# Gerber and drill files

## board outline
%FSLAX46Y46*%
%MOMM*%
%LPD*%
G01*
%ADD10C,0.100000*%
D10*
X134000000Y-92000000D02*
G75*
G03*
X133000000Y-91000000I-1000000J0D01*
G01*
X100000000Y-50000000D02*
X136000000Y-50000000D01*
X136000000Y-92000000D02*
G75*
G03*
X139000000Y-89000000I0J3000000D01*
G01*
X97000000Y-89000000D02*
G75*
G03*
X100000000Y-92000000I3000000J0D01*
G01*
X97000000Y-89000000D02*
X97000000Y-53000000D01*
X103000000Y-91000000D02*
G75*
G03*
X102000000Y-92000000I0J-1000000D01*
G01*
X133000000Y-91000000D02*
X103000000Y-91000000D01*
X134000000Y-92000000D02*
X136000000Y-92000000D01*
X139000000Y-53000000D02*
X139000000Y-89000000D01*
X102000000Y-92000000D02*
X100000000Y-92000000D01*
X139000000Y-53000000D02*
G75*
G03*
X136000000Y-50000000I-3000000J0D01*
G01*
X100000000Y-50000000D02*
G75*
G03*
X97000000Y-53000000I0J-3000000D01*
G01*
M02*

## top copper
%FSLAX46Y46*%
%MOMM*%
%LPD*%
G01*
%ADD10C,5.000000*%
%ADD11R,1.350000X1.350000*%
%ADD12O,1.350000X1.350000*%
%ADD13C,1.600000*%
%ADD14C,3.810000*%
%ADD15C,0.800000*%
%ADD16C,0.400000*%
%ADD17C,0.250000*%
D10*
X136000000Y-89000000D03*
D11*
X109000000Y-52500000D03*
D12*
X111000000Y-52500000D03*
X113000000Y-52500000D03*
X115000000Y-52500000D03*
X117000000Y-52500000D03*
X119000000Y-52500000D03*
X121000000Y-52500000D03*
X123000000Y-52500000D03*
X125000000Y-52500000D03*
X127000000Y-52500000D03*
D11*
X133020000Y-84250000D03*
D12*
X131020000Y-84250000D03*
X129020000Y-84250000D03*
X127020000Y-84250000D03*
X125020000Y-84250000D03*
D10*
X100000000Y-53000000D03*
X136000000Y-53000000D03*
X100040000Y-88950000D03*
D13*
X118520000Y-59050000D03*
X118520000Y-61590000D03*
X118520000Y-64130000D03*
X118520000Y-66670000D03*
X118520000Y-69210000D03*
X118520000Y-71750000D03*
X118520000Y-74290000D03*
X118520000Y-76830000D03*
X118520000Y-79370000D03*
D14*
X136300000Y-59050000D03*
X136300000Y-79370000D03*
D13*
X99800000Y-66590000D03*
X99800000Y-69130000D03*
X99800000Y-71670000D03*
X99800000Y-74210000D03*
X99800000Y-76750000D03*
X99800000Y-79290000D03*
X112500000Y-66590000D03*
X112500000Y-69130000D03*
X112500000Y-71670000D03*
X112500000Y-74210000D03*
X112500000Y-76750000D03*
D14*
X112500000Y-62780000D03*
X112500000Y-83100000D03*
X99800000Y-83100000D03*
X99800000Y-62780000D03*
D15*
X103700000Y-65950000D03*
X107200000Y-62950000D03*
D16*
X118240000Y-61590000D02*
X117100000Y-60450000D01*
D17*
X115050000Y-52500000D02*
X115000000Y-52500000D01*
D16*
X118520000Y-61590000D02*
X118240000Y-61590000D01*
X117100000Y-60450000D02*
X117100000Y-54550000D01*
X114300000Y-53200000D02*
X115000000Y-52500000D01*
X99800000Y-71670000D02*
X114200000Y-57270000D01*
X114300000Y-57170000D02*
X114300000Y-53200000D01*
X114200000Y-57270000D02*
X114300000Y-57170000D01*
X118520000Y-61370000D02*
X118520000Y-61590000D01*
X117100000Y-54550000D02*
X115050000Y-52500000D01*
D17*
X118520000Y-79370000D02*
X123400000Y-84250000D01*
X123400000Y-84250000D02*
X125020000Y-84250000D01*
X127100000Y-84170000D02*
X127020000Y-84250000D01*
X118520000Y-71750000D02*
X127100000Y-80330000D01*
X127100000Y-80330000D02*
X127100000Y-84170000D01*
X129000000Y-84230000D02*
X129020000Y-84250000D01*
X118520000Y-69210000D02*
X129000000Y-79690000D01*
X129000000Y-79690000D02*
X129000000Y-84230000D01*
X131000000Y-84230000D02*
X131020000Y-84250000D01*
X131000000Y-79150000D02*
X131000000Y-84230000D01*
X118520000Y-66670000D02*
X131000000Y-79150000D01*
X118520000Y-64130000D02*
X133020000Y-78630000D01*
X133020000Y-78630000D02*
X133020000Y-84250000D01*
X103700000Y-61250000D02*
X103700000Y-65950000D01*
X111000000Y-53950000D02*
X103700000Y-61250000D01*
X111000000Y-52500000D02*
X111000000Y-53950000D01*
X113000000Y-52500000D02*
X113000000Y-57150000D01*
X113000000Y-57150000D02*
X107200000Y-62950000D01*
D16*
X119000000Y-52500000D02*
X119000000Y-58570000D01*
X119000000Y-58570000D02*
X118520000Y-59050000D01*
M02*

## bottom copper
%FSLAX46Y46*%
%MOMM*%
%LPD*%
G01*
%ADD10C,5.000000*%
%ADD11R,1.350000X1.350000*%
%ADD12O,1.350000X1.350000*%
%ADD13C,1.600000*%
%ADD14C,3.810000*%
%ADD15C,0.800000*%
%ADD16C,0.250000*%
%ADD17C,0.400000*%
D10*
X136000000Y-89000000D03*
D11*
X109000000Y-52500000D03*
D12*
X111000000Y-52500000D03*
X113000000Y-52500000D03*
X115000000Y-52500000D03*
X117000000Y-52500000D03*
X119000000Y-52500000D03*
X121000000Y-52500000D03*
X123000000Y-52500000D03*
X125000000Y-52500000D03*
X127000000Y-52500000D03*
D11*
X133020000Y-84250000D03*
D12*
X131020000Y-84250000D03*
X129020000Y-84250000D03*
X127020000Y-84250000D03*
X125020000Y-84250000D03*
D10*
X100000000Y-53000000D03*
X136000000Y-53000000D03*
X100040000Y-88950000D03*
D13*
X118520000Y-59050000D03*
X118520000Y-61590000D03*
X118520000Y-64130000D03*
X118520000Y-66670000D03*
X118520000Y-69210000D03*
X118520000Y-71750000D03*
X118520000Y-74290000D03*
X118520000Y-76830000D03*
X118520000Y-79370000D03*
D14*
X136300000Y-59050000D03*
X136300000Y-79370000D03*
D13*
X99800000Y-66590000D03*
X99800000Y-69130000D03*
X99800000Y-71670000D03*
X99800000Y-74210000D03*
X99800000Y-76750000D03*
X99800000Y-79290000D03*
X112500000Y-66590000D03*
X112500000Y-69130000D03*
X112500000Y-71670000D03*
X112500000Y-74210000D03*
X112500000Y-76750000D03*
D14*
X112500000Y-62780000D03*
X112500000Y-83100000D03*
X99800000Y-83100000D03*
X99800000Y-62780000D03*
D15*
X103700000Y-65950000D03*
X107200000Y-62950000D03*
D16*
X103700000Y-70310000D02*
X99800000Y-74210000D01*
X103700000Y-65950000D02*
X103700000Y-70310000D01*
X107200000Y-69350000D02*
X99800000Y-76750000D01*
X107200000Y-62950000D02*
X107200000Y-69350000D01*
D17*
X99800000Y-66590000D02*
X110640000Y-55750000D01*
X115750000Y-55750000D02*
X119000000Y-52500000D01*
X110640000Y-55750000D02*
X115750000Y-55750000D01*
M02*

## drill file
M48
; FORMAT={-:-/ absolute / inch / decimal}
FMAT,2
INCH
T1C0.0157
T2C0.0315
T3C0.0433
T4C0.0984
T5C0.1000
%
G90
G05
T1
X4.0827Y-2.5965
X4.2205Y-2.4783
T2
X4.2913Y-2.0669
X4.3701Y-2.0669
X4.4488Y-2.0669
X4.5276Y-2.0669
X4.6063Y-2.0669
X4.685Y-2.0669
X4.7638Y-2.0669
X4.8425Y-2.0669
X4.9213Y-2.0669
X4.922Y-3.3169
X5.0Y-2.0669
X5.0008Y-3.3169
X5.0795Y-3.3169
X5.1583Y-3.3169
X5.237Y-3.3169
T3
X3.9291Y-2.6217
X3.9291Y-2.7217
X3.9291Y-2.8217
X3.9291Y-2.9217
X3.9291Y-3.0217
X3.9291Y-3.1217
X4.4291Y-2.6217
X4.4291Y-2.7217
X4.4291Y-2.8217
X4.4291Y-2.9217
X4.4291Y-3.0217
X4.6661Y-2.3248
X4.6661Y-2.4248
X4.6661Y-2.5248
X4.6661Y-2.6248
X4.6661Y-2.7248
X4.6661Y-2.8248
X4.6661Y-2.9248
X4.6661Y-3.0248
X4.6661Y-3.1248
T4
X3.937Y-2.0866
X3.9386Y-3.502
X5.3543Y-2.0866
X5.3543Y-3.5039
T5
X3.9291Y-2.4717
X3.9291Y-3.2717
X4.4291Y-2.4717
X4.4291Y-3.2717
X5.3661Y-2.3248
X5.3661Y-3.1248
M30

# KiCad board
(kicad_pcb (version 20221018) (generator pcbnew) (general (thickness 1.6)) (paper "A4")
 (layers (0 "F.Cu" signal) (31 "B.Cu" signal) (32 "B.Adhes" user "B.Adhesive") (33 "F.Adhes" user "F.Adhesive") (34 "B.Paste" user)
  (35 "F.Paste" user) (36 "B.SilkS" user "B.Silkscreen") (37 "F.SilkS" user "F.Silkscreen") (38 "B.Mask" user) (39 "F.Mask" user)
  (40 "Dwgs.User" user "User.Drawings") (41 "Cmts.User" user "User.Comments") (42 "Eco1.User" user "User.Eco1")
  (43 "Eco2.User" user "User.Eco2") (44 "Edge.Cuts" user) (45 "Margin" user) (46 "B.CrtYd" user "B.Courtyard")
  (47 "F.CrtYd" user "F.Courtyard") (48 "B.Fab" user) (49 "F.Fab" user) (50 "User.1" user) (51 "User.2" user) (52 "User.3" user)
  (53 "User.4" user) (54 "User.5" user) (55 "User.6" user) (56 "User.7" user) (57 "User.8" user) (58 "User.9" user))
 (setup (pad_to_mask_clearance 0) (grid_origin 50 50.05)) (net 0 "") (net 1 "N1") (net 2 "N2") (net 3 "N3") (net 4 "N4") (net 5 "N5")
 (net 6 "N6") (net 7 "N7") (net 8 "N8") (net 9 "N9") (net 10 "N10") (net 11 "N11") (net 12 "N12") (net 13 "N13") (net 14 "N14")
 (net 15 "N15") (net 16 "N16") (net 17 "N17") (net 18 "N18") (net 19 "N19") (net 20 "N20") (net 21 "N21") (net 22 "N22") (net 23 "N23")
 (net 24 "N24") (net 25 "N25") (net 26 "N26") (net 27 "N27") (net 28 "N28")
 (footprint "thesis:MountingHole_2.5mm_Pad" (layer "F.Cu") (at 136.06 89)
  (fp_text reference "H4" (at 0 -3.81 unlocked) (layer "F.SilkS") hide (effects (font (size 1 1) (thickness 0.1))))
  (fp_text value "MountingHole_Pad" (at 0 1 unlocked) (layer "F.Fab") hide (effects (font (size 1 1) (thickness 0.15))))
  (pad "1" thru_hole circle (at -0.06 0) (size 5 5) (drill 2.5) (layers "*.Cu" "*.Mask") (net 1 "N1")))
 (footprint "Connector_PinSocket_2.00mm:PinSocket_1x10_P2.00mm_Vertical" (layer "F.Cu") (at 109 52.5 90)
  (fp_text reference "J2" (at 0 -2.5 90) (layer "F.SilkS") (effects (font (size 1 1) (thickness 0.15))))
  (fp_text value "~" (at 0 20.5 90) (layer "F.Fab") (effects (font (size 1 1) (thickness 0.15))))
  (pad "1" thru_hole rect (at 0 0 90) (size 1.35 1.35) (drill 0.8) (layers "*.Cu" "*.Mask") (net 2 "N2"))
  (pad "2" thru_hole oval (at 0 2 90) (size 1.35 1.35) (drill 0.8) (layers "*.Cu" "*.Mask") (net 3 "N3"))
  (pad "3" thru_hole oval (at 0 4 90) (size 1.35 1.35) (drill 0.8) (layers "*.Cu" "*.Mask") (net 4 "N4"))
  (pad "4" thru_hole oval (at 0 6 90) (size 1.35 1.35) (drill 0.8) (layers "*.Cu" "*.Mask") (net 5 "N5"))
  (pad "5" thru_hole oval (at 0 8 90) (size 1.35 1.35) (drill 0.8) (layers "*.Cu" "*.Mask") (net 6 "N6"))
  (pad "6" thru_hole oval (at 0 10 90) (size 1.35 1.35) (drill 0.8) (layers "*.Cu" "*.Mask") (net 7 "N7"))
  (pad "7" thru_hole oval (at 0 12 90) (size 1.35 1.35) (drill 0.8) (layers "*.Cu" "*.Mask") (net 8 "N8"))
  (pad "8" thru_hole oval (at 0 14 90) (size 1.35 1.35) (drill 0.8) (layers "*.Cu" "*.Mask") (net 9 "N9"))
  (pad "9" thru_hole oval (at 0 16 90) (size 1.35 1.35) (drill 0.8) (layers "*.Cu" "*.Mask") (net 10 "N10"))
  (pad "10" thru_hole oval (at 0 18 90) (size 1.35 1.35) (drill 0.8) (layers "*.Cu" "*.Mask") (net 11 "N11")))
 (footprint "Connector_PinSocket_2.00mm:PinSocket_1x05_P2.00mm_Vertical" (layer "F.Cu") (at 133.02 84.25 -90)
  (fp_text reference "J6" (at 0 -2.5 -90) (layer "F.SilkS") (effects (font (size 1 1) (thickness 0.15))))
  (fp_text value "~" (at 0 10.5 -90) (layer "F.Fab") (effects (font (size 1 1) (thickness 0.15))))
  (pad "1" thru_hole rect (at 0 0 270) (size 1.35 1.35) (drill 0.8) (layers "*.Cu" "*.Mask") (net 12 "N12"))
  (pad "2" thru_hole oval (at 0 2 270) (size 1.35 1.35) (drill 0.8) (layers "*.Cu" "*.Mask") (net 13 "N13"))
  (pad "3" thru_hole oval (at 0 4 270) (size 1.35 1.35) (drill 0.8) (layers "*.Cu" "*.Mask") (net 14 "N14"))
  (pad "4" thru_hole oval (at 0 6 270) (size 1.35 1.35) (drill 0.8) (layers "*.Cu" "*.Mask") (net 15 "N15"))
  (pad "5" thru_hole oval (at 0 8 270) (size 1.35 1.35) (drill 0.8) (layers "*.Cu" "*.Mask") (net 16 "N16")))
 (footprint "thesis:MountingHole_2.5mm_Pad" (layer "F.Cu") (at 100.06 53)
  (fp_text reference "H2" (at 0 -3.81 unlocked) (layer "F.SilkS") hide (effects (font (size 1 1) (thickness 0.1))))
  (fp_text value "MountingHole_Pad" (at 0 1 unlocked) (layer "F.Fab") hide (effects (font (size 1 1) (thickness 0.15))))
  (pad "1" thru_hole circle (at -0.06 0) (size 5 5) (drill 2.5) (layers "*.Cu" "*.Mask") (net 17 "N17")))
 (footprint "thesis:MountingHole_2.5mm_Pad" (layer "F.Cu") (at 136.06 53)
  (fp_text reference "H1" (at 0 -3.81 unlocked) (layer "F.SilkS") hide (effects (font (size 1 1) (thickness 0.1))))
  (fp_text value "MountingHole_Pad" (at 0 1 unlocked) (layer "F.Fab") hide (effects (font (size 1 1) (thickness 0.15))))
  (pad "1" thru_hole circle (at -0.06 0) (size 5 5) (drill 2.5) (layers "*.Cu" "*.Mask") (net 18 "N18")))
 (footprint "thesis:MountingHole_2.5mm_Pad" (layer "F.Cu") (at 100.1 88.95)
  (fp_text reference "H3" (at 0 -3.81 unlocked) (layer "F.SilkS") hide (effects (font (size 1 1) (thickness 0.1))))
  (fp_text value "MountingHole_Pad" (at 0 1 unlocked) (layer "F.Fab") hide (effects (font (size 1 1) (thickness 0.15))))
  (pad "1" thru_hole circle (at -0.06 0) (size 5 5) (drill 2.5) (layers "*.Cu" "*.Mask") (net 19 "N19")))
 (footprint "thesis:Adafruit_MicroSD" (layer "F.Cu") (at 138.84 56.51 -90)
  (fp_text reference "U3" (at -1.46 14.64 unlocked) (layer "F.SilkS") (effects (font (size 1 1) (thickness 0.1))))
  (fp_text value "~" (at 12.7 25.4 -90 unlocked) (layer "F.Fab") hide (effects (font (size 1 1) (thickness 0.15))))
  (pad "1" thru_hole circle (at 2.54 20.32 270) (size 1.6 1.6) (drill 1.1) (layers "*.Cu" "*.Mask") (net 7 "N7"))
  (pad "2" thru_hole circle (at 5.08 20.32 270) (size 1.6 1.6) (drill 1.1) (layers "*.Cu" "*.Mask") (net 5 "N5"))
  (pad "3" thru_hole circle (at 7.62 20.32 270) (size 1.6 1.6) (drill 1.1) (layers "*.Cu" "*.Mask") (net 12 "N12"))
  (pad "4" thru_hole circle (at 10.16 20.32 270) (size 1.6 1.6) (drill 1.1) (layers "*.Cu" "*.Mask") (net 13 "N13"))
  (pad "5" thru_hole circle (at 12.7 20.32 270) (size 1.6 1.6) (drill 1.1) (layers "*.Cu" "*.Mask") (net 14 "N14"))
  (pad "6" thru_hole circle (at 15.24 20.32 270) (size 1.6 1.6) (drill 1.1) (layers "*.Cu" "*.Mask") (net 15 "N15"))
  (pad "7" thru_hole circle (at 17.78 20.32 270) (size 1.6 1.6) (drill 1.1) (layers "*.Cu" "*.Mask") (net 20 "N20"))
  (pad "8" thru_hole circle (at 20.32 20.32 270) (size 1.6 1.6) (drill 1.1) (layers "*.Cu" "*.Mask") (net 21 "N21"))
  (pad "9" thru_hole circle (at 22.86 20.32 270) (size 1.6 1.6) (drill 1.1) (layers "*.Cu" "*.Mask") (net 16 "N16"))
  (pad "MT1" thru_hole circle (at 2.54 2.54 270) (size 3.81 3.81) (drill 2.54) (layers "*.Cu" "*.Mask"))
  (pad "MT2" thru_hole circle (at 22.86 2.54 270) (size 3.81 3.81) (drill 2.54) (layers "*.Cu" "*.Mask")))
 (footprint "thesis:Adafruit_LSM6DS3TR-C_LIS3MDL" (layer "F.Cu") (at 115.04 60.24 -90)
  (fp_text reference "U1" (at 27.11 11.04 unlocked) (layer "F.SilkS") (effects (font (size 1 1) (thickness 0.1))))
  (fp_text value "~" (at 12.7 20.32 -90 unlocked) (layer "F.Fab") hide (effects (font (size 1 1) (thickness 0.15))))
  (pad "1" thru_hole circle (at 6.35 15.24 270) (size 1.6 1.6) (drill 1.1) (layers "*.Cu" "*.Mask") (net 7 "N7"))
  (pad "2" thru_hole circle (at 8.89 15.24 270) (size 1.6 1.6) (drill 1.1) (layers "*.Cu" "*.Mask") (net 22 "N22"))
  (pad "3" thru_hole circle (at 11.43 15.24 270) (size 1.6 1.6) (drill 1.1) (layers "*.Cu" "*.Mask") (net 5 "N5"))
  (pad "4" thru_hole circle (at 13.97 15.24 270) (size 1.6 1.6) (drill 1.1) (layers "*.Cu" "*.Mask") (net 3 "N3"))
  (pad "5" thru_hole circle (at 16.51 15.24 270) (size 1.6 1.6) (drill 1.1) (layers "*.Cu" "*.Mask") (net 4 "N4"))
  (pad "6" thru_hole circle (at 19.05 15.24 270) (size 1.6 1.6) (drill 1.1) (layers "*.Cu" "*.Mask") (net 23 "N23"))
  (pad "7" thru_hole circle (at 6.35 2.54 270) (size 1.6 1.6) (drill 1.1) (layers "*.Cu" "*.Mask") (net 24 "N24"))
  (pad "8" thru_hole circle (at 8.89 2.54 270) (size 1.6 1.6) (drill 1.1) (layers "*.Cu" "*.Mask") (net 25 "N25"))
  (pad "9" thru_hole circle (at 11.43 2.54 270) (size 1.6 1.6) (drill 1.1) (layers "*.Cu" "*.Mask") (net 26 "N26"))
  (pad "10" thru_hole circle (at 13.97 2.54 270) (size 1.6 1.6) (drill 1.1) (layers "*.Cu" "*.Mask") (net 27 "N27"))
  (pad "11" thru_hole circle (at 16.51 2.54 270) (size 1.6 1.6) (drill 1.1) (layers "*.Cu" "*.Mask") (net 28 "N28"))
  (pad "MH1" thru_hole circle (at 2.54 2.54 270) (size 3.81 3.81) (drill 2.54) (layers "*.Cu" "*.Mask"))
  (pad "MH2" thru_hole circle (at 22.86 2.54 270) (size 3.81 3.81) (drill 2.54) (layers "*.Cu" "*.Mask"))
  (pad "MH3" thru_hole circle (at 22.86 15.24 270) (size 3.81 3.81) (drill 2.54) (layers "*.Cu" "*.Mask"))
  (pad "MH4" thru_hole circle (at 2.54 15.24 270) (size 3.81 3.81) (drill 2.54) (layers "*.Cu" "*.Mask")))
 (gr_arc (start 133 91) (mid 133.707107 91.292893) (end 134 92) (stroke (width 0.1) (type default)) (layer "Edge.Cuts"))
 (gr_line (start 100 50) (end 136 50) (stroke (width 0.1) (type default)) (layer "Edge.Cuts"))
 (gr_arc (start 139 89) (mid 138.12132 91.12132) (end 136 92) (stroke (width 0.1) (type default)) (layer "Edge.Cuts"))
 (gr_arc (start 100 92) (mid 97.87868 91.12132) (end 97 89) (stroke (width 0.1) (type default)) (layer "Edge.Cuts"))
 (gr_line (start 97 89) (end 97 53) (stroke (width 0.1) (type default)) (layer "Edge.Cuts"))
 (gr_arc (start 102 92) (mid 102.292893 91.292893) (end 103 91) (stroke (width 0.1) (type default)) (layer "Edge.Cuts"))
 (gr_line (start 133 91) (end 103 91) (stroke (width 0.1) (type default)) (layer "Edge.Cuts"))
 (gr_line (start 134 92) (end 136 92) (stroke (width 0.1) (type default)) (layer "Edge.Cuts"))
 (gr_line (start 139 53) (end 139 89) (stroke (width 0.1) (type default)) (layer "Edge.Cuts"))
 (gr_line (start 102 92) (end 100 92) (stroke (width 0.1) (type default)) (layer "Edge.Cuts"))
 (gr_arc (start 136 50) (mid 138.12132 50.87868) (end 139 53) (stroke (width 0.1) (type default)) (layer "Edge.Cuts"))
 (gr_arc (start 97 53) (mid 97.87868 50.87868) (end 100 50) (stroke (width 0.1) (type default)) (layer "Edge.Cuts"))
 (segment (start 118.24 61.59) (end 117.1 60.45) (width 0.4) (layer "F.Cu") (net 5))
 (segment (start 115.05 52.5) (end 115 52.5) (width 0.25) (layer "F.Cu") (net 5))
 (segment (start 118.52 61.59) (end 118.24 61.59) (width 0.4) (layer "F.Cu") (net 5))
 (segment (start 117.1 60.45) (end 117.1 54.55) (width 0.4) (layer "F.Cu") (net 5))
 (segment (start 114.3 53.2) (end 115 52.5) (width 0.4) (layer "F.Cu") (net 5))
 (segment (start 99.8 71.67) (end 114.2 57.27) (width 0.4) (layer "F.Cu") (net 5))
 (segment (start 114.3 57.17) (end 114.3 53.2) (width 0.4) (layer "F.Cu") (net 5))
 (segment (start 114.2 57.27) (end 114.3 57.17) (width 0.4) (layer "F.Cu") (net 5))
 (segment (start 118.52 61.37) (end 118.52 61.59) (width 0.4) (layer "F.Cu") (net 5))
 (segment (start 117.1 54.55) (end 115.05 52.5) (width 0.4) (layer "F.Cu") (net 5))
 (segment (start 118.52 79.37) (end 123.4 84.25) (width 0.25) (layer "F.Cu") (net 16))
 (segment (start 123.4 84.25) (end 125.02 84.25) (width 0.25) (layer "F.Cu") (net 16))
 (segment (start 127.1 84.17) (end 127.02 84.25) (width 0.25) (layer "F.Cu") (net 15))
 (segment (start 118.52 71.75) (end 127.1 80.33) (width 0.25) (layer "F.Cu") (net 15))
 (segment (start 127.1 80.33) (end 127.1 84.17) (width 0.25) (layer "F.Cu") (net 15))
 (segment (start 129 84.23) (end 129.02 84.25) (width 0.25) (layer "F.Cu") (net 14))
 (segment (start 118.52 69.21) (end 129 79.69) (width 0.25) (layer "F.Cu") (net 14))
 (segment (start 129 79.69) (end 129 84.23) (width 0.25) (layer "F.Cu") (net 14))
 (segment (start 131 84.23) (end 131.02 84.25) (width 0.25) (layer "F.Cu") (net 13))
 (segment (start 131 79.15) (end 131 84.23) (width 0.25) (layer "F.Cu") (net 13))
 (segment (start 118.52 66.67) (end 131 79.15) (width 0.25) (layer "F.Cu") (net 13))
 (segment (start 118.52 64.13) (end 133.02 78.63) (width 0.25) (layer "F.Cu") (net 12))
 (segment (start 133.02 78.63) (end 133.02 84.25) (width 0.25) (layer "F.Cu") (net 12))
 (segment (start 103.7 61.25) (end 103.7 65.95) (width 0.25) (layer "F.Cu") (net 3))
 (segment (start 111 53.95) (end 103.7 61.25) (width 0.25) (layer "F.Cu") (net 3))
 (segment (start 111 52.5) (end 111 53.95) (width 0.25) (layer "F.Cu") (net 3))
 (via (at 103.7 65.95) (size 0.8) (drill 0.4) (layers "F.Cu" "B.Cu") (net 3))
 (segment (start 103.7 70.31) (end 99.8 74.21) (width 0.25) (layer "B.Cu") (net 3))
 (segment (start 103.7 65.95) (end 103.7 70.31) (width 0.25) (layer "B.Cu") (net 3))
 (segment (start 113 52.5) (end 113 57.15) (width 0.25) (layer "F.Cu") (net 4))
 (segment (start 113 57.15) (end 107.2 62.95) (width 0.25) (layer "F.Cu") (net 4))
 (via (at 107.2 62.95) (size 0.8) (drill 0.4) (layers "F.Cu" "B.Cu") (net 4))
 (segment (start 107.2 69.35) (end 99.8 76.75) (width 0.25) (layer "B.Cu") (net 4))
 (segment (start 107.2 62.95) (end 107.2 69.35) (width 0.25) (layer "B.Cu") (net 4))
 (segment (start 119 52.5) (end 119 58.57) (width 0.4) (layer "F.Cu") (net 7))
 (segment (start 119 58.57) (end 118.52 59.05) (width 0.4) (layer "F.Cu") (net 7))
 (segment (start 99.8 66.59) (end 110.64 55.75) (width 0.4) (layer "B.Cu") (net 7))
 (segment (start 115.75 55.75) (end 119 52.5) (width 0.4) (layer "B.Cu") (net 7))
 (segment (start 110.64 55.75) (end 115.75 55.75) (width 0.4) (layer "B.Cu") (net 7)))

